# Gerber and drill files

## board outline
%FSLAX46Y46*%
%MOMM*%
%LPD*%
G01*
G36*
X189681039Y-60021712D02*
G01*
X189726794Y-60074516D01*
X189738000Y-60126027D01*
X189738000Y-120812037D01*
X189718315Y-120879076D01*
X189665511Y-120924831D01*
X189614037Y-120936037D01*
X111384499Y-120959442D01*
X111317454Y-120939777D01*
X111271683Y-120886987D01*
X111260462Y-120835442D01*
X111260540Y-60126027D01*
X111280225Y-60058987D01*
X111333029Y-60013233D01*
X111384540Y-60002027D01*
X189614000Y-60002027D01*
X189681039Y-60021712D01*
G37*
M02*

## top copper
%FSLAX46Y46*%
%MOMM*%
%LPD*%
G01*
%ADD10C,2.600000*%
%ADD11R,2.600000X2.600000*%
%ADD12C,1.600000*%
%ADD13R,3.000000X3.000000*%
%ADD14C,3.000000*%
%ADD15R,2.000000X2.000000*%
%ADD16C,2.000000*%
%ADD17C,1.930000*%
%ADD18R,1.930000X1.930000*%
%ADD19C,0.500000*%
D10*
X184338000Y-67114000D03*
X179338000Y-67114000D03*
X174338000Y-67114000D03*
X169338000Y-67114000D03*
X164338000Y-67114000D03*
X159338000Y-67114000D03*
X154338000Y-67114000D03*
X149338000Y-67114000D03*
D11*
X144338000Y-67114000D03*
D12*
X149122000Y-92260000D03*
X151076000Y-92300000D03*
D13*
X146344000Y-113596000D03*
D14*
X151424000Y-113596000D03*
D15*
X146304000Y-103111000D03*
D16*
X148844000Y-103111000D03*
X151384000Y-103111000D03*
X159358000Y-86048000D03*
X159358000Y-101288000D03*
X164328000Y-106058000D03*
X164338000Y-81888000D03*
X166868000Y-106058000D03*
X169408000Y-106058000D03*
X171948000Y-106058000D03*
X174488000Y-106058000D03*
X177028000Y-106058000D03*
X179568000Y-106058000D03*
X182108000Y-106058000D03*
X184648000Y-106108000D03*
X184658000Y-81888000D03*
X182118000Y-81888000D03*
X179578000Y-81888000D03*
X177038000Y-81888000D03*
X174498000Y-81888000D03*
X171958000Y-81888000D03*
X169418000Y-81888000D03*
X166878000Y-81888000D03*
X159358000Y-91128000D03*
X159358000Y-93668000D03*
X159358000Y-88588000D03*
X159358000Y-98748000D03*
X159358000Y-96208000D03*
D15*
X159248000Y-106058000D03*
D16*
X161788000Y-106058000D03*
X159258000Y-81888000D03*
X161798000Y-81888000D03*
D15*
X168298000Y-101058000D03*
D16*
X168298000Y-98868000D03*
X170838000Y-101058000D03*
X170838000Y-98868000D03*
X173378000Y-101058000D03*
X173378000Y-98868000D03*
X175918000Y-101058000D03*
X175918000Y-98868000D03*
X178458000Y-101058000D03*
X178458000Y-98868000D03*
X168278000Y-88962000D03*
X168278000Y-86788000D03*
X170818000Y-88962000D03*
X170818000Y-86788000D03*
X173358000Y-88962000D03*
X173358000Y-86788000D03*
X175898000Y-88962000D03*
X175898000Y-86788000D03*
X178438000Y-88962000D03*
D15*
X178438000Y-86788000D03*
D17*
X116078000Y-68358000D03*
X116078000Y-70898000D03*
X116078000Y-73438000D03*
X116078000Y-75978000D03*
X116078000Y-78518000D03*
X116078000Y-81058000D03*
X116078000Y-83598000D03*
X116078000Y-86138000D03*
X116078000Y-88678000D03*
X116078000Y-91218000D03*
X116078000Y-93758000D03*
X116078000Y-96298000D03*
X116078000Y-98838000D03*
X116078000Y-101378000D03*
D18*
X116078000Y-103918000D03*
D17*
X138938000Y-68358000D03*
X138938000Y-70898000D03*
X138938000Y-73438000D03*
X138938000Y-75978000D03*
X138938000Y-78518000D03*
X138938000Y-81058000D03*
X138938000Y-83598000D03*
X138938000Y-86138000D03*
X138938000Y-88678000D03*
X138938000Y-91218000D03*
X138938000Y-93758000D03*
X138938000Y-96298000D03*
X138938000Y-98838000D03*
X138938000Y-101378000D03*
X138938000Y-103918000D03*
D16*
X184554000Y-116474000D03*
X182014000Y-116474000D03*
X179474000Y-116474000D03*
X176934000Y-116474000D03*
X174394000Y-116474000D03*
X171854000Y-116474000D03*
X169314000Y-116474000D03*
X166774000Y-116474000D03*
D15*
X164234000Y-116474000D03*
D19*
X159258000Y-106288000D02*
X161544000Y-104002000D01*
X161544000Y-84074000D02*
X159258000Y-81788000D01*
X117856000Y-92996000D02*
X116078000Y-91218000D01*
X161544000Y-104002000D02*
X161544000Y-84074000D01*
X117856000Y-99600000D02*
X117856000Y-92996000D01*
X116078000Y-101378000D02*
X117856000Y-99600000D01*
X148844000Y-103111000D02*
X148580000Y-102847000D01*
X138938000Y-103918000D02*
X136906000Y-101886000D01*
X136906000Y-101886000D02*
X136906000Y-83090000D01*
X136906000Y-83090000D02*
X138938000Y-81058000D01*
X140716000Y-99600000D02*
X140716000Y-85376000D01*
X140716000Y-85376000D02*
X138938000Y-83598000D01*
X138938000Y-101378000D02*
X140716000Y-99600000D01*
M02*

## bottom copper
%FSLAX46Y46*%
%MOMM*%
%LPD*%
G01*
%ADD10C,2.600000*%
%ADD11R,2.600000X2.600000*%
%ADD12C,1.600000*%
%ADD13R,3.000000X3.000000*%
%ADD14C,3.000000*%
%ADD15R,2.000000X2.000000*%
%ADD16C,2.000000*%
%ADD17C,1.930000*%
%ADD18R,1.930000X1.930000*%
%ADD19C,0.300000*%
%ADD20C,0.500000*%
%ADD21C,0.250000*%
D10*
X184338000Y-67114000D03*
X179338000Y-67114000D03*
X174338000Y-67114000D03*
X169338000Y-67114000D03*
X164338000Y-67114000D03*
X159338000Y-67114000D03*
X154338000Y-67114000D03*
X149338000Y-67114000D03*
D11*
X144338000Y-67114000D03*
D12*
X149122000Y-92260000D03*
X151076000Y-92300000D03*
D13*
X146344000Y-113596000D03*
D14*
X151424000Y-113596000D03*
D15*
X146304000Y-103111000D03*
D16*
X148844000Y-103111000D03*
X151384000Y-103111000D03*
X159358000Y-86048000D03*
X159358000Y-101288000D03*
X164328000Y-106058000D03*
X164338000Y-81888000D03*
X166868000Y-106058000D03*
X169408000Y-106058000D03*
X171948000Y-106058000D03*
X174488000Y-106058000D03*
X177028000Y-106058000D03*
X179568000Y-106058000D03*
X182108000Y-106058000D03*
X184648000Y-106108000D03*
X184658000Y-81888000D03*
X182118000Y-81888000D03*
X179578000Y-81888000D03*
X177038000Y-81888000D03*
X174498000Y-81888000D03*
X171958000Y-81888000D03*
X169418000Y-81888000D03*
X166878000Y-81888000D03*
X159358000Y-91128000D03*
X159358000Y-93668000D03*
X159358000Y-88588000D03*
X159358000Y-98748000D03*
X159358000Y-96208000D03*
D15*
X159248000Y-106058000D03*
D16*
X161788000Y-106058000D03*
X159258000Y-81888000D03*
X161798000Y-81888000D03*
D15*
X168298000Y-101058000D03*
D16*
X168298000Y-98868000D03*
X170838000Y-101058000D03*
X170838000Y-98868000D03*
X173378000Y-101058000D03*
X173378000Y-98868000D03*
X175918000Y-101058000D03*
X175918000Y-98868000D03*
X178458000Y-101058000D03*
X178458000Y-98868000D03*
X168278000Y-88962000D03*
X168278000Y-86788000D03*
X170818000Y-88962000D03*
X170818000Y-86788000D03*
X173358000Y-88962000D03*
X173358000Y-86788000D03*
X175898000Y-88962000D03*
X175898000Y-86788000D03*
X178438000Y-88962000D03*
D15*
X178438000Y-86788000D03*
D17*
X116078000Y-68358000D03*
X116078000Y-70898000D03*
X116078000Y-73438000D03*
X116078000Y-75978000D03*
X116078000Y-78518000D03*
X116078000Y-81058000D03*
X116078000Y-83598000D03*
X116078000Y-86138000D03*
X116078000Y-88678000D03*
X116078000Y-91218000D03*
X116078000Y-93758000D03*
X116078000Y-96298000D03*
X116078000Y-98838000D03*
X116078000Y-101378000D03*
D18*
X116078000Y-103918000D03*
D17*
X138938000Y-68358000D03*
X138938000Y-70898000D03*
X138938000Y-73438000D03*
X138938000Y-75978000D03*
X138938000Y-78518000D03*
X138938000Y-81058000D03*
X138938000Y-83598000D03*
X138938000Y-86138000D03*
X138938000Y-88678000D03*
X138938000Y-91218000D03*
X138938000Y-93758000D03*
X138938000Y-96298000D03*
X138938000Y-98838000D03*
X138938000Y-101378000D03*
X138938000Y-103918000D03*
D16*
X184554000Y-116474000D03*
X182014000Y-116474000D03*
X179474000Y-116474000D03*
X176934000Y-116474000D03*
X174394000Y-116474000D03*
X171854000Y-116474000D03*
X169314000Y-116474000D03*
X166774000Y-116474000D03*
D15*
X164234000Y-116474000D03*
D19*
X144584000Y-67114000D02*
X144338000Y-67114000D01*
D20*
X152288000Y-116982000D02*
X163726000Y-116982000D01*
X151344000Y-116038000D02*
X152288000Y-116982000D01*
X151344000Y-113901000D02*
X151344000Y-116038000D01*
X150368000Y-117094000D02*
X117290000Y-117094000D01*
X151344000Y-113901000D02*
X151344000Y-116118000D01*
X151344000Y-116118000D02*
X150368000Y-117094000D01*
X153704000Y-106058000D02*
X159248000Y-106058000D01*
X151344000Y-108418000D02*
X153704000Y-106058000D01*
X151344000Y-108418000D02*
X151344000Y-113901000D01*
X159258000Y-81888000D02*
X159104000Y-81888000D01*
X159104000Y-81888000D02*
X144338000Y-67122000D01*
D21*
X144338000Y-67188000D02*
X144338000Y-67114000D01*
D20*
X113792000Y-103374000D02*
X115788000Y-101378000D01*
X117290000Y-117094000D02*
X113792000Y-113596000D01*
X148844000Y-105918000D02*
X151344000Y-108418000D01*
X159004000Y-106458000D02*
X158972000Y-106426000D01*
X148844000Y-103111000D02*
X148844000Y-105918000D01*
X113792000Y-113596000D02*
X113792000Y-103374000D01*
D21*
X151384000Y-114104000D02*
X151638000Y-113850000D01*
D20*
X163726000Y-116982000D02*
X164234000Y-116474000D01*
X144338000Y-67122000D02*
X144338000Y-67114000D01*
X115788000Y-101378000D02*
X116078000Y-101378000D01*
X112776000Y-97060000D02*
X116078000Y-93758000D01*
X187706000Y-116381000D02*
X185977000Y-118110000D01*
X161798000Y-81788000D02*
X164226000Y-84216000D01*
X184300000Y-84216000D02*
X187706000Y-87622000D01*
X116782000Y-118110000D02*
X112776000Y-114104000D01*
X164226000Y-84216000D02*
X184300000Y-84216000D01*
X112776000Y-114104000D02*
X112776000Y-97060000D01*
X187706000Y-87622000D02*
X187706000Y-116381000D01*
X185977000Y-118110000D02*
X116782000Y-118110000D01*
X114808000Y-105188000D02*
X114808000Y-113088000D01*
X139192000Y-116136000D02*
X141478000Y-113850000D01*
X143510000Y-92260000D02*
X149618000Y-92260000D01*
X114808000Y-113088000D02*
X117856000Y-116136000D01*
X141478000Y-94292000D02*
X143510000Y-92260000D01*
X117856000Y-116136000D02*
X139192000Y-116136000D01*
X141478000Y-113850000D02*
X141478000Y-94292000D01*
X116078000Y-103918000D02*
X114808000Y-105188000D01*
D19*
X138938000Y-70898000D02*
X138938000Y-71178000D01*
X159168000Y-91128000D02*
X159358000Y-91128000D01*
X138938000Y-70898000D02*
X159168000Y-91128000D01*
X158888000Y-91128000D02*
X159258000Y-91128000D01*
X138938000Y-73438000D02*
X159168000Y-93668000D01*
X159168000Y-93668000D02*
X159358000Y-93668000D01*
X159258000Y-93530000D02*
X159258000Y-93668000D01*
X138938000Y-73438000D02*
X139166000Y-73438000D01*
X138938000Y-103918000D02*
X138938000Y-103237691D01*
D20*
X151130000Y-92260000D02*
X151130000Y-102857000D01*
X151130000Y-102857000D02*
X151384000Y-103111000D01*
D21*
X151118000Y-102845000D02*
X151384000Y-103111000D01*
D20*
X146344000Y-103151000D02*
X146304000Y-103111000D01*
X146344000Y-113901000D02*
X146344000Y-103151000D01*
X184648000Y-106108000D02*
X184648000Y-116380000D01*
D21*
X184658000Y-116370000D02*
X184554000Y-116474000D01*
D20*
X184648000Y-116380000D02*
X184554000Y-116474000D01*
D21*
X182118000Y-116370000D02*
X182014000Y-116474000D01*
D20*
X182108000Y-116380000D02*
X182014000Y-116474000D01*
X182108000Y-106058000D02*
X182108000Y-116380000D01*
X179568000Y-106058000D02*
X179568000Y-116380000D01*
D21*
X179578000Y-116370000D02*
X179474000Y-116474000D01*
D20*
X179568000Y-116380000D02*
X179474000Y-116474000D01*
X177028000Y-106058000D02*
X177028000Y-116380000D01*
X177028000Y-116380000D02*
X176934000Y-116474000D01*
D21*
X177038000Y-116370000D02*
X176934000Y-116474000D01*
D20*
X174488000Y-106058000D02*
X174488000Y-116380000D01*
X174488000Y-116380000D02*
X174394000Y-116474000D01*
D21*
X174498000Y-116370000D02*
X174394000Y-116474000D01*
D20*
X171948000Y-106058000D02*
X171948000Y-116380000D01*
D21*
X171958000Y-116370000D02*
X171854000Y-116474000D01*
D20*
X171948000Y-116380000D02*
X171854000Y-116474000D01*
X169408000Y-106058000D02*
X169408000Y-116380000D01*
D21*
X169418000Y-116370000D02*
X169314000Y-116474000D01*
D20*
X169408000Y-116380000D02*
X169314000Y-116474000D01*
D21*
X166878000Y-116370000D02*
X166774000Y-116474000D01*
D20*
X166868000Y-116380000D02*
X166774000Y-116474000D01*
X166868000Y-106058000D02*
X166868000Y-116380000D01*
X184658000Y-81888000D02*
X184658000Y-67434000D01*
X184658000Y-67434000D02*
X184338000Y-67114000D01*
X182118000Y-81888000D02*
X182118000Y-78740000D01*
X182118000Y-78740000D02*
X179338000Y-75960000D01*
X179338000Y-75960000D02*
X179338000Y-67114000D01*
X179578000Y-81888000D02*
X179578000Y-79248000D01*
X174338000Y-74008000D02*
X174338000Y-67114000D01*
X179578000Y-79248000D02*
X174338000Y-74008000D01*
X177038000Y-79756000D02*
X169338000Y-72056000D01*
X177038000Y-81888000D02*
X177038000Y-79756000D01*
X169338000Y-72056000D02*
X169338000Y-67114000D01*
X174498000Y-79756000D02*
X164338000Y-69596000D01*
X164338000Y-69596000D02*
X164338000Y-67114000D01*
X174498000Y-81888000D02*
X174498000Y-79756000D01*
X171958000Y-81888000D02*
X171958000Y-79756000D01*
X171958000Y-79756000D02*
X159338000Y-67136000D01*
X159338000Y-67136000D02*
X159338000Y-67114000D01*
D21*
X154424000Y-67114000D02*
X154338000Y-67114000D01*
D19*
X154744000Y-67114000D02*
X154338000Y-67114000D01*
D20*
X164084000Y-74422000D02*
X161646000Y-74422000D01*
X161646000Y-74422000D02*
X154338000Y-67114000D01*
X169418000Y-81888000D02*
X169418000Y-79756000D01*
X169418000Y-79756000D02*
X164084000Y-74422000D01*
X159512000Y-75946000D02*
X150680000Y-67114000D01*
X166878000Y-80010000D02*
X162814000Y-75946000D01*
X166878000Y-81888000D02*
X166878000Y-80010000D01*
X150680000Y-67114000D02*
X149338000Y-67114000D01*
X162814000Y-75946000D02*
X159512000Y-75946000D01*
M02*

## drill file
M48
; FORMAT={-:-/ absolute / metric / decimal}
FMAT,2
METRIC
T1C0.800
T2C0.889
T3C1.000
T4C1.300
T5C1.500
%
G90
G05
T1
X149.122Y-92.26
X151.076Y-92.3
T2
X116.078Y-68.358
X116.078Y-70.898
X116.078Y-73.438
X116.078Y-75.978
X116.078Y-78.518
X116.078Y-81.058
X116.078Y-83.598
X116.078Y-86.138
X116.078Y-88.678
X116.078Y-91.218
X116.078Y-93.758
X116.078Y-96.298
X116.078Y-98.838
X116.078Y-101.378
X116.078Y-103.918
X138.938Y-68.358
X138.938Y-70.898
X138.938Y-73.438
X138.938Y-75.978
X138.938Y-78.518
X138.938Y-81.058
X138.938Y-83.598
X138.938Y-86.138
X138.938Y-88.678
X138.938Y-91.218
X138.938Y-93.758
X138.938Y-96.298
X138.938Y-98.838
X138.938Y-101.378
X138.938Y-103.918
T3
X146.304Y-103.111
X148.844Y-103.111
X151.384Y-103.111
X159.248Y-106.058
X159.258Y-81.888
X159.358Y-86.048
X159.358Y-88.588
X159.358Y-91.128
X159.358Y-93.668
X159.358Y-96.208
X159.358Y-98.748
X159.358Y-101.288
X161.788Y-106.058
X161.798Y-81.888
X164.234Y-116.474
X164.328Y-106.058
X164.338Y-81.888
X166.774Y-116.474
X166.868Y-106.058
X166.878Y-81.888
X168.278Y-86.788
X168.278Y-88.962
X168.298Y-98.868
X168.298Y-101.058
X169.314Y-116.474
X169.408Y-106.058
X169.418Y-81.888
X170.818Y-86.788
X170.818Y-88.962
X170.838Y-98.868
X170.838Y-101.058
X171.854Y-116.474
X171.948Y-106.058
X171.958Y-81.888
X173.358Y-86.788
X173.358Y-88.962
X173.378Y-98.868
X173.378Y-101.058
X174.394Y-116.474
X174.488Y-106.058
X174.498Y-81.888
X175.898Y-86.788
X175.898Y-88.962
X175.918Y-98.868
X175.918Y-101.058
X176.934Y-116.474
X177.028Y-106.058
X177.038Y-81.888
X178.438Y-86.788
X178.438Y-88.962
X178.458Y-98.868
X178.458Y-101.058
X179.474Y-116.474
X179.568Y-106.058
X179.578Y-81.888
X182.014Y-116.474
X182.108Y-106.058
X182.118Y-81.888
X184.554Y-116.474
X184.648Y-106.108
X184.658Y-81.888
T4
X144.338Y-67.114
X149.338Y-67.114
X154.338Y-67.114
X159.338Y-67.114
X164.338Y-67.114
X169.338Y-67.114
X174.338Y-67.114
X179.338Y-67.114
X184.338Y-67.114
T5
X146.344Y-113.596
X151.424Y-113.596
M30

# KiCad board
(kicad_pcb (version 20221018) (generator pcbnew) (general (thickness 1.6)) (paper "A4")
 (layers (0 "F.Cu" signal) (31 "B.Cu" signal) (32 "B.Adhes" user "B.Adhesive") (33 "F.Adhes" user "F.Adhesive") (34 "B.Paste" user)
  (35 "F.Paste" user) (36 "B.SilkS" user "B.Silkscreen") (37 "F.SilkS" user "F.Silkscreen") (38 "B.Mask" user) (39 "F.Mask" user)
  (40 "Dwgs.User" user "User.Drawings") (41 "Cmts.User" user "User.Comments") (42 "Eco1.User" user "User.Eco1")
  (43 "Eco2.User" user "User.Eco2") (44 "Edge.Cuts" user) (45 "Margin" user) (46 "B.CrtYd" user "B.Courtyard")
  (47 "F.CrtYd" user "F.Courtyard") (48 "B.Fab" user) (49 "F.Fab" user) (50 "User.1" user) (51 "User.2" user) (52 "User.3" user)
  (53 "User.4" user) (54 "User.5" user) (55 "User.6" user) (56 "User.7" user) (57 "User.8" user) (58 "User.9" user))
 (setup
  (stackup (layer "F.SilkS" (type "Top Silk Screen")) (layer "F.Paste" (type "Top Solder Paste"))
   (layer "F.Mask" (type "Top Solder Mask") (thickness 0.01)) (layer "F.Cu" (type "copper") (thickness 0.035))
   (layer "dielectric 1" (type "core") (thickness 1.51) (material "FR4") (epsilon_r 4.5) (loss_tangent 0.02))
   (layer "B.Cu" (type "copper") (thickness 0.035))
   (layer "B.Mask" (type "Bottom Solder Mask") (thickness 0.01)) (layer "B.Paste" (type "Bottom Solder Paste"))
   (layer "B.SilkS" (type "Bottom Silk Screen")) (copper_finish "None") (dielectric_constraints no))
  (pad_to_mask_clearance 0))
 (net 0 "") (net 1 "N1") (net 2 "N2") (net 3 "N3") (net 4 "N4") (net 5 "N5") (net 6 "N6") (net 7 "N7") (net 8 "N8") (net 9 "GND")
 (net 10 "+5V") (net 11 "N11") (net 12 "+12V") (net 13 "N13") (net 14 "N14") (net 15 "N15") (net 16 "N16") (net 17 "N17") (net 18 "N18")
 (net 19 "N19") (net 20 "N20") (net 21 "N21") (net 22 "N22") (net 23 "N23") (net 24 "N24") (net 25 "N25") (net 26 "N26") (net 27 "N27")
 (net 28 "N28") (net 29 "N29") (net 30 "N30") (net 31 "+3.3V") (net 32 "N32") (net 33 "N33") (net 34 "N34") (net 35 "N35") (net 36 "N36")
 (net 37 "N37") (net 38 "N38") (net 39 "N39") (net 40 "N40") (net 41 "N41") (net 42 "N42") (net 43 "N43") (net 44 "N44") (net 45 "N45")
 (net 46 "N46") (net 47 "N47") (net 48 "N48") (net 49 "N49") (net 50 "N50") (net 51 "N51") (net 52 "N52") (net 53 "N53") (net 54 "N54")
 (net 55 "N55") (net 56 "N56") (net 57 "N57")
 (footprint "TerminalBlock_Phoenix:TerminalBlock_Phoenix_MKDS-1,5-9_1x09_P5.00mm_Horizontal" (layer "F.Cu") (at 184.338 67.114 180)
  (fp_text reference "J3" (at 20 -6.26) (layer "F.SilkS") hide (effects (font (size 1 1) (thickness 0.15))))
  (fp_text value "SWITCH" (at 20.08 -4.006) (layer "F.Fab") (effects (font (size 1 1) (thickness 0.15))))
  (pad "1" thru_hole circle (at 0 0 180) (size 2.6 2.6) (drill 1.3) (layers "*.Cu" "*.Mask") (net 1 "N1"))
  (pad "2" thru_hole circle (at 5 0 180) (size 2.6 2.6) (drill 1.3) (layers "*.Cu" "*.Mask") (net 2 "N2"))
  (pad "3" thru_hole circle (at 10 0 180) (size 2.6 2.6) (drill 1.3) (layers "*.Cu" "*.Mask") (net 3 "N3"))
  (pad "4" thru_hole circle (at 15 0 180) (size 2.6 2.6) (drill 1.3) (layers "*.Cu" "*.Mask") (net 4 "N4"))
  (pad "5" thru_hole circle (at 20 0 180) (size 2.6 2.6) (drill 1.3) (layers "*.Cu" "*.Mask") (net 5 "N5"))
  (pad "6" thru_hole circle (at 25 0 180) (size 2.6 2.6) (drill 1.3) (layers "*.Cu" "*.Mask") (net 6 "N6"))
  (pad "7" thru_hole circle (at 30 0 180) (size 2.6 2.6) (drill 1.3) (layers "*.Cu" "*.Mask") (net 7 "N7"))
  (pad "8" thru_hole circle (at 35 0 180) (size 2.6 2.6) (drill 1.3) (layers "*.Cu" "*.Mask") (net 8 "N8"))
  (pad "9" thru_hole rect (at 40 0 180) (size 2.6 2.6) (drill 1.3) (layers "*.Cu" "*.Mask") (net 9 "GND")))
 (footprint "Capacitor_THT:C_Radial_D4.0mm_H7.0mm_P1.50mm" (layer "F.Cu") (at 149.376 92.26)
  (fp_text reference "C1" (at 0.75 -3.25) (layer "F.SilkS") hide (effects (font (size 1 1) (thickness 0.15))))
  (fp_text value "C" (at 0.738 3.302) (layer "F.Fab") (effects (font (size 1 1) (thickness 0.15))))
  (pad "1" thru_hole circle (at -0.254 0) (size 1.6 1.6) (drill 0.8) (layers "*.Cu" "*.Mask") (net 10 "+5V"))
  (pad "2" thru_hole circle (at 1.7 0.04) (size 1.6 1.6) (drill 0.8) (layers "*.Cu" "*.Mask") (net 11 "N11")))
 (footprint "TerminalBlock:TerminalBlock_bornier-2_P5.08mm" (layer "F.Cu") (at 146.344 113.596)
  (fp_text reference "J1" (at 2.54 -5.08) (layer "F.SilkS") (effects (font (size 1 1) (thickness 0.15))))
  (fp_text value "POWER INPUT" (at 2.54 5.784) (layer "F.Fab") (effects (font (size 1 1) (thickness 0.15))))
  (pad "1" thru_hole rect (at 0 0) (size 3 3) (drill 1.5) (layers "*.Cu" "*.Mask") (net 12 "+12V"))
  (pad "2" thru_hole circle (at 5.08 0) (size 3 3) (drill 1.5) (layers "*.Cu" "*.Mask") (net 9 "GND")))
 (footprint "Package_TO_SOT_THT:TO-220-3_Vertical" (layer "F.Cu") (at 146.304 103.111)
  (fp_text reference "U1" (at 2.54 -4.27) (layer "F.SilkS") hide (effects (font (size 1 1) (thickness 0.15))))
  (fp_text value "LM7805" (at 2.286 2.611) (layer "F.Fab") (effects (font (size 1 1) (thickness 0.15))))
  (pad "1" thru_hole rect (at 0 0) (size 2 2) (drill 1) (layers "*.Cu" "*.Mask") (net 12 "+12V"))
  (pad "2" thru_hole circle (at 2.54 0) (size 2 2) (drill 1) (layers "*.Cu" "*.Mask") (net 9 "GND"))
  (pad "3" thru_hole circle (at 5.08 0) (size 2 2) (drill 1) (layers "*.Cu" "*.Mask") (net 11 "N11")))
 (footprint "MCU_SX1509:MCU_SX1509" (layer "F.Cu") (at 172.258 93.788 90)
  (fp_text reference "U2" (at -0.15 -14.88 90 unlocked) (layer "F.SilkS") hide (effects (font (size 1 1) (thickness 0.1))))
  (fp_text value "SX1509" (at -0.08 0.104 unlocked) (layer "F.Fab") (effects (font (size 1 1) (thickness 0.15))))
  (pad "0" thru_hole circle (at 7.74 -12.9 90) (size 2 2) (drill 1) (layers "*.Cu" "*.Mask") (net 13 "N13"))
  (pad "1" thru_hole circle (at -7.5 -12.9 90) (size 2 2) (drill 1) (layers "*.Cu" "*.Mask") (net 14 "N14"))
  (pad "2" thru_hole circle (at -12.27 -7.93 90) (size 2 2) (drill 1) (layers "*.Cu" "*.Mask") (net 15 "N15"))
  (pad "3" thru_hole circle (at 11.9 -7.92 90) (size 2 2) (drill 1) (layers "*.Cu" "*.Mask") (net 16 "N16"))
  (pad "4" thru_hole circle (at -12.27 -5.39 90) (size 2 2) (drill 1) (layers "*.Cu" "*.Mask") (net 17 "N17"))
  (pad "5" thru_hole circle (at -12.27 -2.85 90) (size 2 2) (drill 1) (layers "*.Cu" "*.Mask") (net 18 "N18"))
  (pad "6" thru_hole circle (at -12.27 -0.31 90) (size 2 2) (drill 1) (layers "*.Cu" "*.Mask") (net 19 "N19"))
  (pad "7" thru_hole circle (at -12.27 2.23 90) (size 2 2) (drill 1) (layers "*.Cu" "*.Mask") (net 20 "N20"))
  (pad "8" thru_hole circle (at -12.27 4.77 90) (size 2 2) (drill 1) (layers "*.Cu" "*.Mask") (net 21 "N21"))
  (pad "9" thru_hole circle (at -12.27 7.31 90) (size 2 2) (drill 1) (layers "*.Cu" "*.Mask") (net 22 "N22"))
  (pad "10" thru_hole circle (at -12.27 9.85 90) (size 2 2) (drill 1) (layers "*.Cu" "*.Mask") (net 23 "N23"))
  (pad "11" thru_hole circle (at -12.32 12.39 90) (size 2 2) (drill 1) (layers "*.Cu" "*.Mask") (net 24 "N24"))
  (pad "12" thru_hole circle (at 11.9 12.4 90) (size 2 2) (drill 1) (layers "*.Cu" "*.Mask") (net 1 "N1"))
  (pad "13" thru_hole circle (at 11.9 9.86 90) (size 2 2) (drill 1) (layers "*.Cu" "*.Mask") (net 2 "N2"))
  (pad "14" thru_hole circle (at 11.9 7.32 90) (size 2 2) (drill 1) (layers "*.Cu" "*.Mask") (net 3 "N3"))
  (pad "15" thru_hole circle (at 11.9 4.78 90) (size 2 2) (drill 1) (layers "*.Cu" "*.Mask") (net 4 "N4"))
  (pad "16" thru_hole circle (at 11.9 2.24 90) (size 2 2) (drill 1) (layers "*.Cu" "*.Mask") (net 5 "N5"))
  (pad "17" thru_hole circle (at 11.9 -0.3 90) (size 2 2) (drill 1) (layers "*.Cu" "*.Mask") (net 6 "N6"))
  (pad "18" thru_hole circle (at 11.9 -2.84 90) (size 2 2) (drill 1) (layers "*.Cu" "*.Mask") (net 7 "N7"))
  (pad "19" thru_hole circle (at 11.9 -5.38 90) (size 2 2) (drill 1) (layers "*.Cu" "*.Mask") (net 8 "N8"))
  (pad "20" thru_hole circle (at 2.66 -12.9 90) (size 2 2) (drill 1) (layers "*.Cu" "*.Mask") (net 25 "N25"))
  (pad "21" thru_hole circle (at 0.12 -12.9 90) (size 2 2) (drill 1) (layers "*.Cu" "*.Mask") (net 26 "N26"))
  (pad "22" thru_hole circle (at 5.2 -12.9 90) (size 2 2) (drill 1) (layers "*.Cu" "*.Mask") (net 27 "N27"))
  (pad "23" thru_hole circle (at -4.96 -12.9 90) (size 2 2) (drill 1) (layers "*.Cu" "*.Mask") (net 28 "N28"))
  (pad "24" thru_hole circle (at -2.42 -12.9 90) (size 2 2) (drill 1) (layers "*.Cu" "*.Mask") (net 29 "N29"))
  (pad "25" thru_hole rect (at -12.27 -13.01 90) (size 2 2) (drill 1) (layers "*.Cu" "*.Mask") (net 9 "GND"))
  (pad "26" thru_hole circle (at -12.27 -10.47 90) (size 2 2) (drill 1) (layers "*.Cu" "*.Mask") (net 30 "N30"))
  (pad "27" thru_hole circle (at 11.9 -13 90) (size 2 2) (drill 1) (layers "*.Cu" "*.Mask") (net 9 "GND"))
  (pad "28" thru_hole circle (at 11.9 -10.46 90) (size 2 2) (drill 1) (layers "*.Cu" "*.Mask") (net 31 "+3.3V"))
  (pad "29" thru_hole rect (at -7.27 -3.96 90) (size 2 2) (drill 1) (layers "*.Cu" "*.Mask"))
  (pad "30" thru_hole circle (at -5.08 -3.96 90) (size 2 2) (drill 1) (layers "*.Cu" "*.Mask"))
  (pad "31" thru_hole circle (at -7.27 -1.42 90) (size 2 2) (drill 1) (layers "*.Cu" "*.Mask"))
  (pad "32" thru_hole circle (at -5.08 -1.42 90) (size 2 2) (drill 1) (layers "*.Cu" "*.Mask"))
  (pad "33" thru_hole circle (at -7.27 1.12 90) (size 2 2) (drill 1) (layers "*.Cu" "*.Mask") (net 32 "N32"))
  (pad "34" thru_hole circle (at -5.08 1.12 90) (size 2 2) (drill 1) (layers "*.Cu" "*.Mask") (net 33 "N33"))
  (pad "35" thru_hole circle (at -7.27 3.66 90) (size 2 2) (drill 1) (layers "*.Cu" "*.Mask"))
  (pad "36" thru_hole circle (at -5.08 3.66 90) (size 2 2) (drill 1) (layers "*.Cu" "*.Mask"))
  (pad "37" thru_hole circle (at -7.27 6.2 90) (size 2 2) (drill 1) (layers "*.Cu" "*.Mask"))
  (pad "38" thru_hole circle (at -5.08 6.2 90) (size 2 2) (drill 1) (layers "*.Cu" "*.Mask"))
  (pad "39" thru_hole circle (at 4.826 -3.98 90) (size 2 2) (drill 1) (layers "*.Cu" "*.Mask"))
  (pad "40" thru_hole circle (at 7 -3.98 90) (size 2 2) (drill 1) (layers "*.Cu" "*.Mask"))
  (pad "41" thru_hole circle (at 4.826 -1.44 90) (size 2 2) (drill 1) (layers "*.Cu" "*.Mask"))
  (pad "42" thru_hole circle (at 7 -1.44 90) (size 2 2) (drill 1) (layers "*.Cu" "*.Mask"))
  (pad "43" thru_hole circle (at 4.826 1.1 90) (size 2 2) (drill 1) (layers "*.Cu" "*.Mask") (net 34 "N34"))
  (pad "44" thru_hole circle (at 7 1.1 90) (size 2 2) (drill 1) (layers "*.Cu" "*.Mask") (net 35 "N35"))
  (pad "45" thru_hole circle (at 4.826 3.64 90) (size 2 2) (drill 1) (layers "*.Cu" "*.Mask"))
  (pad "46" thru_hole circle (at 7 3.64 90) (size 2 2) (drill 1) (layers "*.Cu" "*.Mask"))
  (pad "47" thru_hole circle (at 4.826 6.18 90) (size 2 2) (drill 1) (layers "*.Cu" "*.Mask"))
  (pad "48" thru_hole rect (at 7 6.18 90) (size 2 2) (drill 1) (layers "*.Cu" "*.Mask")))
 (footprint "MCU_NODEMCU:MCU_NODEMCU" (layer "F.Cu") (at 127.508 86.138)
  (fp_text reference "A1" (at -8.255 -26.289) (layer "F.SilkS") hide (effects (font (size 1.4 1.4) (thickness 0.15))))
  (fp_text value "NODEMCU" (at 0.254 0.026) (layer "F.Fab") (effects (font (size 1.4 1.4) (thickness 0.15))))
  (pad "J1_1" thru_hole circle (at -11.43 -17.78) (size 1.93 1.93) (drill 0.889) (layers "*.Cu" "*.Mask") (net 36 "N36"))
  (pad "J1_2" thru_hole circle (at -11.43 -15.24) (size 1.93 1.93) (drill 0.889) (layers "*.Cu" "*.Mask") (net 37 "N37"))
  (pad "J1_3" thru_hole circle (at -11.43 -12.7) (size 1.93 1.93) (drill 0.889) (layers "*.Cu" "*.Mask") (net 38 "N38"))
  (pad "J1_4" thru_hole circle (at -11.43 -10.16) (size 1.93 1.93) (drill 0.889) (layers "*.Cu" "*.Mask") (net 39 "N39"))
  (pad "J1_5" thru_hole circle (at -11.43 -7.62) (size 1.93 1.93) (drill 0.889) (layers "*.Cu" "*.Mask") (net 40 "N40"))
  (pad "J1_6" thru_hole circle (at -11.43 -5.08) (size 1.93 1.93) (drill 0.889) (layers "*.Cu" "*.Mask") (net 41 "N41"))
  (pad "J1_7" thru_hole circle (at -11.43 -2.54) (size 1.93 1.93) (drill 0.889) (layers "*.Cu" "*.Mask") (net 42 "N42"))
  (pad "J1_8" thru_hole circle (at -11.43 0) (size 1.93 1.93) (drill 0.889) (layers "*.Cu" "*.Mask") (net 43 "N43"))
  (pad "J1_9" thru_hole circle (at -11.43 2.54) (size 1.93 1.93) (drill 0.889) (layers "*.Cu" "*.Mask") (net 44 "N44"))
  (pad "J1_10" thru_hole circle (at -11.43 5.08) (size 1.93 1.93) (drill 0.889) (layers "*.Cu" "*.Mask") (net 9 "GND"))
  (pad "J1_11" thru_hole circle (at -11.43 7.62) (size 1.93 1.93) (drill 0.889) (layers "*.Cu" "*.Mask") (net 31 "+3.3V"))
  (pad "J1_12" thru_hole circle (at -11.43 10.16) (size 1.93 1.93) (drill 0.889) (layers "*.Cu" "*.Mask") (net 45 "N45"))
  (pad "J1_13" thru_hole circle (at -11.43 12.7) (size 1.93 1.93) (drill 0.889) (layers "*.Cu" "*.Mask") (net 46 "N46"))
  (pad "J1_14" thru_hole circle (at -11.43 15.24) (size 1.93 1.93) (drill 0.889) (layers "*.Cu" "*.Mask") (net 9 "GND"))
  (pad "J1_15" thru_hole rect (at -11.43 17.78) (size 1.93 1.93) (drill 0.889) (layers "*.Cu" "*.Mask") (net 10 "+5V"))
  (pad "J2_1" thru_hole circle (at 11.43 -17.78) (size 1.93 1.93) (drill 0.889) (layers "*.Cu" "*.Mask") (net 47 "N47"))
  (pad "J2_2" thru_hole circle (at 11.43 -15.24) (size 1.93 1.93) (drill 0.889) (layers "*.Cu" "*.Mask") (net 25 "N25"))
  (pad "J2_3" thru_hole circle (at 11.43 -12.7) (size 1.93 1.93) (drill 0.889) (layers "*.Cu" "*.Mask") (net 26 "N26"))
  (pad "J2_4" thru_hole circle (at 11.43 -10.16) (size 1.93 1.93) (drill 0.889) (layers "*.Cu" "*.Mask") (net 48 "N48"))
  (pad "J2_5" thru_hole circle (at 11.43 -7.62) (size 1.93 1.93) (drill 0.889) (layers "*.Cu" "*.Mask") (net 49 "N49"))
  (pad "J2_6" thru_hole circle (at 11.43 -5.08) (size 1.93 1.93) (drill 0.889) (layers "*.Cu" "*.Mask") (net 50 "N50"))
  (pad "J2_7" thru_hole circle (at 11.43 -2.54) (size 1.93 1.93) (drill 0.889) (layers "*.Cu" "*.Mask") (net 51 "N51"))
  (pad "J2_8" thru_hole circle (at 11.43 0) (size 1.93 1.93) (drill 0.889) (layers "*.Cu" "*.Mask") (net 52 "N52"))
  (pad "J2_9" thru_hole circle (at 11.43 2.54) (size 1.93 1.93) (drill 0.889) (layers "*.Cu" "*.Mask") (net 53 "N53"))
  (pad "J2_10" thru_hole circle (at 11.43 5.08) (size 1.93 1.93) (drill 0.889) (layers "*.Cu" "*.Mask") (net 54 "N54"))
  (pad "J2_11" thru_hole circle (at 11.43 7.62) (size 1.93 1.93) (drill 0.889) (layers "*.Cu" "*.Mask") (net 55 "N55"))
  (pad "J2_12" thru_hole circle (at 11.43 10.16) (size 1.93 1.93) (drill 0.889) (layers "*.Cu" "*.Mask") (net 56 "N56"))
  (pad "J2_13" thru_hole circle (at 11.43 12.7) (size 1.93 1.93) (drill 0.889) (layers "*.Cu" "*.Mask") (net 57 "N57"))
  (pad "J2_14" thru_hole circle (at 11.43 15.24) (size 1.93 1.93) (drill 0.889) (layers "*.Cu" "*.Mask") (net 51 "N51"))
  (pad "J2_15" thru_hole circle (at 11.43 17.78) (size 1.93 1.93) (drill 0.889) (layers "*.Cu" "*.Mask") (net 50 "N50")))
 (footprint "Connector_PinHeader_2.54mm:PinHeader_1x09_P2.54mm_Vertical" (layer "F.Cu") (at 184.554 116.474 -90)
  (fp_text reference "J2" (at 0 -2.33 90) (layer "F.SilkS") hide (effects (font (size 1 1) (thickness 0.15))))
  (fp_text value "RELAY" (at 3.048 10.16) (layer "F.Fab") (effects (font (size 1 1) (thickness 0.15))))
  (pad "1" thru_hole circle (at 0 0 270) (size 2 2) (drill 1) (layers "*.Cu" "*.Mask") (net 24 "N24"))
  (pad "2" thru_hole circle (at 0 2.54 270) (size 2 2) (drill 1) (layers "*.Cu" "*.Mask") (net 23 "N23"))
  (pad "3" thru_hole circle (at 0 5.08 270) (size 2 2) (drill 1) (layers "*.Cu" "*.Mask") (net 22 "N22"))
  (pad "4" thru_hole circle (at 0 7.62 270) (size 2 2) (drill 1) (layers "*.Cu" "*.Mask") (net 21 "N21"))
  (pad "5" thru_hole circle (at 0 10.16 270) (size 2 2) (drill 1) (layers "*.Cu" "*.Mask") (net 20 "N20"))
  (pad "6" thru_hole circle (at 0 12.7 270) (size 2 2) (drill 1) (layers "*.Cu" "*.Mask") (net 19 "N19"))
  (pad "7" thru_hole circle (at 0 15.24 270) (size 2 2) (drill 1) (layers "*.Cu" "*.Mask") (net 18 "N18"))
  (pad "8" thru_hole circle (at 0 17.78 270) (size 2 2) (drill 1) (layers "*.Cu" "*.Mask") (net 17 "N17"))
  (pad "9" thru_hole rect (at 0 20.32 270) (size 2 2) (drill 1) (layers "*.Cu" "*.Mask") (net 9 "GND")))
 (segment (start 159.258 106.288) (end 161.544 104.002) (width 0.5) (layer "F.Cu") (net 9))
 (segment (start 161.544 84.074) (end 159.258 81.788) (width 0.5) (layer "F.Cu") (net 9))
 (segment (start 117.856 92.996) (end 116.078 91.218) (width 0.5) (layer "F.Cu") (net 9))
 (segment (start 161.544 104.002) (end 161.544 84.074) (width 0.5) (layer "F.Cu") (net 9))
 (segment (start 117.856 99.6) (end 117.856 92.996) (width 0.5) (layer "F.Cu") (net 9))
 (segment (start 116.078 101.378) (end 117.856 99.6) (width 0.5) (layer "F.Cu") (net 9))
 (segment (start 148.844 103.111) (end 148.58 102.847) (width 0.5) (layer "F.Cu") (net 9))
 (segment (start 144.584 67.114) (end 144.338 67.114) (width 0.3) (layer "B.Cu") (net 9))
 (segment (start 152.288 116.982) (end 163.726 116.982) (width 0.5) (layer "B.Cu") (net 9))
 (segment (start 151.344 116.038) (end 152.288 116.982) (width 0.5) (layer "B.Cu") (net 9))
 (segment (start 151.344 113.901) (end 151.344 116.038) (width 0.5) (layer "B.Cu") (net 9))
 (segment (start 150.368 117.094) (end 117.29 117.094) (width 0.5) (layer "B.Cu") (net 9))
 (segment (start 151.344 113.901) (end 151.344 116.118) (width 0.5) (layer "B.Cu") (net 9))
 (segment (start 151.344 116.118) (end 150.368 117.094) (width 0.5) (layer "B.Cu") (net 9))
 (segment (start 153.704 106.058) (end 159.248 106.058) (width 0.5) (layer "B.Cu") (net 9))
 (segment (start 151.344 108.418) (end 153.704 106.058) (width 0.5) (layer "B.Cu") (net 9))
 (segment (start 151.344 108.418) (end 151.344 113.901) (width 0.5) (layer "B.Cu") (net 9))
 (segment (start 159.258 81.888) (end 159.104 81.888) (width 0.5) (layer "B.Cu") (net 9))
 (segment (start 159.104 81.888) (end 144.338 67.122) (width 0.5) (layer "B.Cu") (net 9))
 (segment (start 144.338 67.188) (end 144.338 67.114) (width 0.25) (layer "B.Cu") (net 9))
 (segment (start 113.792 103.374) (end 115.788 101.378) (width 0.5) (layer "B.Cu") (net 9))
 (segment (start 117.29 117.094) (end 113.792 113.596) (width 0.5) (layer "B.Cu") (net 9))
 (segment (start 148.844 105.918) (end 151.344 108.418) (width 0.5) (layer "B.Cu") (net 9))
 (segment (start 159.004 106.458) (end 158.972 106.426) (width 0.5) (layer "B.Cu") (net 9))
 (segment (start 148.844 103.111) (end 148.844 105.918) (width 0.5) (layer "B.Cu") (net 9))
 (segment (start 113.792 113.596) (end 113.792 103.374) (width 0.5) (layer "B.Cu") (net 9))
 (segment (start 151.384 114.104) (end 151.638 113.85) (width 0.25) (layer "B.Cu") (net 9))
 (segment (start 163.726 116.982) (end 164.234 116.474) (width 0.5) (layer "B.Cu") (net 9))
 (segment (start 144.338 67.122) (end 144.338 67.114) (width 0.5) (layer "B.Cu") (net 9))
 (segment (start 115.788 101.378) (end 116.078 101.378) (width 0.5) (layer "B.Cu") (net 9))
 (segment (start 112.776 97.06) (end 116.078 93.758) (width 0.5) (layer "B.Cu") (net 31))
 (segment (start 187.706 116.381) (end 185.977 118.11) (width 0.5) (layer "B.Cu") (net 31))
 (segment (start 161.798 81.788) (end 164.226 84.216) (width 0.5) (layer "B.Cu") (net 31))
 (segment (start 184.3 84.216) (end 187.706 87.622) (width 0.5) (layer "B.Cu") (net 31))
 (segment (start 116.782 118.11) (end 112.776 114.104) (width 0.5) (layer "B.Cu") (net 31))
 (segment (start 164.226 84.216) (end 184.3 84.216) (width 0.5) (layer "B.Cu") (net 31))
 (segment (start 112.776 114.104) (end 112.776 97.06) (width 0.5) (layer "B.Cu") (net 31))
 (segment (start 187.706 87.622) (end 187.706 116.381) (width 0.5) (layer "B.Cu") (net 31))
 (segment (start 185.977 118.11) (end 116.782 118.11) (width 0.5) (layer "B.Cu") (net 31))
 (segment (start 114.808 105.188) (end 114.808 113.088) (width 0.5) (layer "B.Cu") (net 10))
 (segment (start 139.192 116.136) (end 141.478 113.85) (width 0.5) (layer "B.Cu") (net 10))
 (segment (start 143.51 92.26) (end 149.618 92.26) (width 0.5) (layer "B.Cu") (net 10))
 (segment (start 114.808 113.088) (end 117.856 116.136) (width 0.5) (layer "B.Cu") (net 10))
 (segment (start 141.478 94.292) (end 143.51 92.26) (width 0.5) (layer "B.Cu") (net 10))
 (segment (start 117.856 116.136) (end 139.192 116.136) (width 0.5) (layer "B.Cu") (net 10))
 (segment (start 141.478 113.85) (end 141.478 94.292) (width 0.5) (layer "B.Cu") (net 10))
 (segment (start 116.078 103.918) (end 114.808 105.188) (width 0.5) (layer "B.Cu") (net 10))
 (segment (start 138.938 70.898) (end 138.938 71.178) (width 0.3) (layer "B.Cu") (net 25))
 (segment (start 159.168 91.128) (end 159.358 91.128) (width 0.3) (layer "B.Cu") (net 25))
 (segment (start 138.938 70.898) (end 159.168 91.128) (width 0.3) (layer "B.Cu") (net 25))
 (segment (start 158.888 91.128) (end 159.258 91.128) (width 0.3) (layer "B.Cu") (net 25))
 (segment (start 138.938 73.438) (end 159.168 93.668) (width 0.3) (layer "B.Cu") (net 26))
 (segment (start 159.168 93.668) (end 159.358 93.668) (width 0.3) (layer "B.Cu") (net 26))
 (segment (start 159.258 93.53) (end 159.258 93.668) (width 0.3) (layer "B.Cu") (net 26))
 (segment (start 138.938 73.438) (end 139.166 73.438) (width 0.3) (layer "B.Cu") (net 26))
 (segment (start 138.938 103.918) (end 136.906 101.886) (width 0.5) (layer "F.Cu") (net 50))
 (segment (start 136.906 101.886) (end 136.906 83.09) (width 0.5) (layer "F.Cu") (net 50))
 (segment (start 136.906 83.09) (end 138.938 81.058) (width 0.5) (layer "F.Cu") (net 50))
 (segment (start 138.938 103.918) (end 138.938 103.237691) (width 0.3) (layer "B.Cu") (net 50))
 (segment (start 140.716 99.6) (end 140.716 85.376) (width 0.5) (layer "F.Cu") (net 51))
 (segment (start 140.716 85.376) (end 138.938 83.598) (width 0.5) (layer "F.Cu") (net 51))
 (segment (start 138.938 101.378) (end 140.716 99.6) (width 0.5) (layer "F.Cu") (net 51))
 (segment (start 151.13 92.26) (end 151.13 102.857) (width 0.5) (layer "B.Cu") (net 11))
 (segment (start 151.13 102.857) (end 151.384 103.111) (width 0.5) (layer "B.Cu") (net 11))
 (segment (start 151.118 102.845) (end 151.384 103.111) (width 0.25) (layer "B.Cu") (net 11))
 (segment (start 146.344 103.151) (end 146.304 103.111) (width 0.5) (layer "B.Cu") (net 12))
 (segment (start 146.344 113.901) (end 146.344 103.151) (width 0.5) (layer "B.Cu") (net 12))
 (segment (start 184.648 106.108) (end 184.648 116.38) (width 0.5) (layer "B.Cu") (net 24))
 (segment (start 184.658 116.37) (end 184.554 116.474) (width 0.25) (layer "B.Cu") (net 24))
 (segment (start 184.648 116.38) (end 184.554 116.474) (width 0.5) (layer "B.Cu") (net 24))
 (segment (start 182.118 116.37) (end 182.014 116.474) (width 0.25) (layer "B.Cu") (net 23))
 (segment (start 182.108 116.38) (end 182.014 116.474) (width 0.5) (layer "B.Cu") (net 23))
 (segment (start 182.108 106.058) (end 182.108 116.38) (width 0.5) (layer "B.Cu") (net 23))
 (segment (start 179.568 106.058) (end 179.568 116.38) (width 0.5) (layer "B.Cu") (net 22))
 (segment (start 179.578 116.37) (end 179.474 116.474) (width 0.25) (layer "B.Cu") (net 22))
 (segment (start 179.568 116.38) (end 179.474 116.474) (width 0.5) (layer "B.Cu") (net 22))
 (segment (start 177.028 106.058) (end 177.028 116.38) (width 0.5) (layer "B.Cu") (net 21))
 (segment (start 177.028 116.38) (end 176.934 116.474) (width 0.5) (layer "B.Cu") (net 21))
 (segment (start 177.038 116.37) (end 176.934 116.474) (width 0.25) (layer "B.Cu") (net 21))
 (segment (start 174.488 106.058) (end 174.488 116.38) (width 0.5) (layer "B.Cu") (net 20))
 (segment (start 174.488 116.38) (end 174.394 116.474) (width 0.5) (layer "B.Cu") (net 20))
 (segment (start 174.498 116.37) (end 174.394 116.474) (width 0.25) (layer "B.Cu") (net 20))
 (segment (start 171.948 106.058) (end 171.948 116.38) (width 0.5) (layer "B.Cu") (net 19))
 (segment (start 171.958 116.37) (end 171.854 116.474) (width 0.25) (layer "B.Cu") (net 19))
 (segment (start 171.948 116.38) (end 171.854 116.474) (width 0.5) (layer "B.Cu") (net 19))
 (segment (start 169.408 106.058) (end 169.408 116.38) (width 0.5) (layer "B.Cu") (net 18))
 (segment (start 169.418 116.37) (end 169.314 116.474) (width 0.25) (layer "B.Cu") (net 18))
 (segment (start 169.408 116.38) (end 169.314 116.474) (width 0.5) (layer "B.Cu") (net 18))
 (segment (start 166.878 116.37) (end 166.774 116.474) (width 0.25) (layer "B.Cu") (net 17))
 (segment (start 166.868 116.38) (end 166.774 116.474) (width 0.5) (layer "B.Cu") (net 17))
 (segment (start 166.868 106.058) (end 166.868 116.38) (width 0.5) (layer "B.Cu") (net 17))
 (segment (start 184.658 81.888) (end 184.658 67.434) (width 0.5) (layer "B.Cu") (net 1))
 (segment (start 184.658 67.434) (end 184.338 67.114) (width 0.5) (layer "B.Cu") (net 1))
 (segment (start 182.118 81.888) (end 182.118 78.74) (width 0.5) (layer "B.Cu") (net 2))
 (segment (start 182.118 78.74) (end 179.338 75.96) (width 0.5) (layer "B.Cu") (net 2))
 (segment (start 179.338 75.96) (end 179.338 67.114) (width 0.5) (layer "B.Cu") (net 2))
 (segment (start 179.578 81.888) (end 179.578 79.248) (width 0.5) (layer "B.Cu") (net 3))
 (segment (start 174.338 74.008) (end 174.338 67.114) (width 0.5) (layer "B.Cu") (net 3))
 (segment (start 179.578 79.248) (end 174.338 74.008) (width 0.5) (layer "B.Cu") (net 3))
 (segment (start 177.038 79.756) (end 169.338 72.056) (width 0.5) (layer "B.Cu") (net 4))
 (segment (start 177.038 81.888) (end 177.038 79.756) (width 0.5) (layer "B.Cu") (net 4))
 (segment (start 169.338 72.056) (end 169.338 67.114) (width 0.5) (layer "B.Cu") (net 4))
 (segment (start 174.498 79.756) (end 164.338 69.596) (width 0.5) (layer "B.Cu") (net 5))
 (segment (start 164.338 69.596) (end 164.338 67.114) (width 0.5) (layer "B.Cu") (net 5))
 (segment (start 174.498 81.888) (end 174.498 79.756) (width 0.5) (layer "B.Cu") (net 5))
 (segment (start 171.958 81.888) (end 171.958 79.756) (width 0.5) (layer "B.Cu") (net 6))
 (segment (start 171.958 79.756) (end 159.338 67.136) (width 0.5) (layer "B.Cu") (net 6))
 (segment (start 159.338 67.136) (end 159.338 67.114) (width 0.5) (layer "B.Cu") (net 6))
 (segment (start 154.424 67.114) (end 154.338 67.114) (width 0.25) (layer "B.Cu") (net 7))
 (segment (start 154.744 67.114) (end 154.338 67.114) (width 0.3) (layer "B.Cu") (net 7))
 (segment (start 164.084 74.422) (end 161.646 74.422) (width 0.5) (layer "B.Cu") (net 7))
 (segment (start 161.646 74.422) (end 154.338 67.114) (width 0.5) (layer "B.Cu") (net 7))
 (segment (start 169.418 81.888) (end 169.418 79.756) (width 0.5) (layer "B.Cu") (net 7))
 (segment (start 169.418 79.756) (end 164.084 74.422) (width 0.5) (layer "B.Cu") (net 7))
 (segment (start 159.512 75.946) (end 150.68 67.114) (width 0.5) (layer "B.Cu") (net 8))
 (segment (start 166.878 80.01) (end 162.814 75.946) (width 0.5) (layer "B.Cu") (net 8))
 (segment (start 166.878 81.888) (end 166.878 80.01) (width 0.5) (layer "B.Cu") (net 8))
 (segment (start 150.68 67.114) (end 149.338 67.114) (width 0.5) (layer "B.Cu") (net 8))
 (segment (start 162.814 75.946) (end 159.512 75.946) (width 0.5) (layer "B.Cu") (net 8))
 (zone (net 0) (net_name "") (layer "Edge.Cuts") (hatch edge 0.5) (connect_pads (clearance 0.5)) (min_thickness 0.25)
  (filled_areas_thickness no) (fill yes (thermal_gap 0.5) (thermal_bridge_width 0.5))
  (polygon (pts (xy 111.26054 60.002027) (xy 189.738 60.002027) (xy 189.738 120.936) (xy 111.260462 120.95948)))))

